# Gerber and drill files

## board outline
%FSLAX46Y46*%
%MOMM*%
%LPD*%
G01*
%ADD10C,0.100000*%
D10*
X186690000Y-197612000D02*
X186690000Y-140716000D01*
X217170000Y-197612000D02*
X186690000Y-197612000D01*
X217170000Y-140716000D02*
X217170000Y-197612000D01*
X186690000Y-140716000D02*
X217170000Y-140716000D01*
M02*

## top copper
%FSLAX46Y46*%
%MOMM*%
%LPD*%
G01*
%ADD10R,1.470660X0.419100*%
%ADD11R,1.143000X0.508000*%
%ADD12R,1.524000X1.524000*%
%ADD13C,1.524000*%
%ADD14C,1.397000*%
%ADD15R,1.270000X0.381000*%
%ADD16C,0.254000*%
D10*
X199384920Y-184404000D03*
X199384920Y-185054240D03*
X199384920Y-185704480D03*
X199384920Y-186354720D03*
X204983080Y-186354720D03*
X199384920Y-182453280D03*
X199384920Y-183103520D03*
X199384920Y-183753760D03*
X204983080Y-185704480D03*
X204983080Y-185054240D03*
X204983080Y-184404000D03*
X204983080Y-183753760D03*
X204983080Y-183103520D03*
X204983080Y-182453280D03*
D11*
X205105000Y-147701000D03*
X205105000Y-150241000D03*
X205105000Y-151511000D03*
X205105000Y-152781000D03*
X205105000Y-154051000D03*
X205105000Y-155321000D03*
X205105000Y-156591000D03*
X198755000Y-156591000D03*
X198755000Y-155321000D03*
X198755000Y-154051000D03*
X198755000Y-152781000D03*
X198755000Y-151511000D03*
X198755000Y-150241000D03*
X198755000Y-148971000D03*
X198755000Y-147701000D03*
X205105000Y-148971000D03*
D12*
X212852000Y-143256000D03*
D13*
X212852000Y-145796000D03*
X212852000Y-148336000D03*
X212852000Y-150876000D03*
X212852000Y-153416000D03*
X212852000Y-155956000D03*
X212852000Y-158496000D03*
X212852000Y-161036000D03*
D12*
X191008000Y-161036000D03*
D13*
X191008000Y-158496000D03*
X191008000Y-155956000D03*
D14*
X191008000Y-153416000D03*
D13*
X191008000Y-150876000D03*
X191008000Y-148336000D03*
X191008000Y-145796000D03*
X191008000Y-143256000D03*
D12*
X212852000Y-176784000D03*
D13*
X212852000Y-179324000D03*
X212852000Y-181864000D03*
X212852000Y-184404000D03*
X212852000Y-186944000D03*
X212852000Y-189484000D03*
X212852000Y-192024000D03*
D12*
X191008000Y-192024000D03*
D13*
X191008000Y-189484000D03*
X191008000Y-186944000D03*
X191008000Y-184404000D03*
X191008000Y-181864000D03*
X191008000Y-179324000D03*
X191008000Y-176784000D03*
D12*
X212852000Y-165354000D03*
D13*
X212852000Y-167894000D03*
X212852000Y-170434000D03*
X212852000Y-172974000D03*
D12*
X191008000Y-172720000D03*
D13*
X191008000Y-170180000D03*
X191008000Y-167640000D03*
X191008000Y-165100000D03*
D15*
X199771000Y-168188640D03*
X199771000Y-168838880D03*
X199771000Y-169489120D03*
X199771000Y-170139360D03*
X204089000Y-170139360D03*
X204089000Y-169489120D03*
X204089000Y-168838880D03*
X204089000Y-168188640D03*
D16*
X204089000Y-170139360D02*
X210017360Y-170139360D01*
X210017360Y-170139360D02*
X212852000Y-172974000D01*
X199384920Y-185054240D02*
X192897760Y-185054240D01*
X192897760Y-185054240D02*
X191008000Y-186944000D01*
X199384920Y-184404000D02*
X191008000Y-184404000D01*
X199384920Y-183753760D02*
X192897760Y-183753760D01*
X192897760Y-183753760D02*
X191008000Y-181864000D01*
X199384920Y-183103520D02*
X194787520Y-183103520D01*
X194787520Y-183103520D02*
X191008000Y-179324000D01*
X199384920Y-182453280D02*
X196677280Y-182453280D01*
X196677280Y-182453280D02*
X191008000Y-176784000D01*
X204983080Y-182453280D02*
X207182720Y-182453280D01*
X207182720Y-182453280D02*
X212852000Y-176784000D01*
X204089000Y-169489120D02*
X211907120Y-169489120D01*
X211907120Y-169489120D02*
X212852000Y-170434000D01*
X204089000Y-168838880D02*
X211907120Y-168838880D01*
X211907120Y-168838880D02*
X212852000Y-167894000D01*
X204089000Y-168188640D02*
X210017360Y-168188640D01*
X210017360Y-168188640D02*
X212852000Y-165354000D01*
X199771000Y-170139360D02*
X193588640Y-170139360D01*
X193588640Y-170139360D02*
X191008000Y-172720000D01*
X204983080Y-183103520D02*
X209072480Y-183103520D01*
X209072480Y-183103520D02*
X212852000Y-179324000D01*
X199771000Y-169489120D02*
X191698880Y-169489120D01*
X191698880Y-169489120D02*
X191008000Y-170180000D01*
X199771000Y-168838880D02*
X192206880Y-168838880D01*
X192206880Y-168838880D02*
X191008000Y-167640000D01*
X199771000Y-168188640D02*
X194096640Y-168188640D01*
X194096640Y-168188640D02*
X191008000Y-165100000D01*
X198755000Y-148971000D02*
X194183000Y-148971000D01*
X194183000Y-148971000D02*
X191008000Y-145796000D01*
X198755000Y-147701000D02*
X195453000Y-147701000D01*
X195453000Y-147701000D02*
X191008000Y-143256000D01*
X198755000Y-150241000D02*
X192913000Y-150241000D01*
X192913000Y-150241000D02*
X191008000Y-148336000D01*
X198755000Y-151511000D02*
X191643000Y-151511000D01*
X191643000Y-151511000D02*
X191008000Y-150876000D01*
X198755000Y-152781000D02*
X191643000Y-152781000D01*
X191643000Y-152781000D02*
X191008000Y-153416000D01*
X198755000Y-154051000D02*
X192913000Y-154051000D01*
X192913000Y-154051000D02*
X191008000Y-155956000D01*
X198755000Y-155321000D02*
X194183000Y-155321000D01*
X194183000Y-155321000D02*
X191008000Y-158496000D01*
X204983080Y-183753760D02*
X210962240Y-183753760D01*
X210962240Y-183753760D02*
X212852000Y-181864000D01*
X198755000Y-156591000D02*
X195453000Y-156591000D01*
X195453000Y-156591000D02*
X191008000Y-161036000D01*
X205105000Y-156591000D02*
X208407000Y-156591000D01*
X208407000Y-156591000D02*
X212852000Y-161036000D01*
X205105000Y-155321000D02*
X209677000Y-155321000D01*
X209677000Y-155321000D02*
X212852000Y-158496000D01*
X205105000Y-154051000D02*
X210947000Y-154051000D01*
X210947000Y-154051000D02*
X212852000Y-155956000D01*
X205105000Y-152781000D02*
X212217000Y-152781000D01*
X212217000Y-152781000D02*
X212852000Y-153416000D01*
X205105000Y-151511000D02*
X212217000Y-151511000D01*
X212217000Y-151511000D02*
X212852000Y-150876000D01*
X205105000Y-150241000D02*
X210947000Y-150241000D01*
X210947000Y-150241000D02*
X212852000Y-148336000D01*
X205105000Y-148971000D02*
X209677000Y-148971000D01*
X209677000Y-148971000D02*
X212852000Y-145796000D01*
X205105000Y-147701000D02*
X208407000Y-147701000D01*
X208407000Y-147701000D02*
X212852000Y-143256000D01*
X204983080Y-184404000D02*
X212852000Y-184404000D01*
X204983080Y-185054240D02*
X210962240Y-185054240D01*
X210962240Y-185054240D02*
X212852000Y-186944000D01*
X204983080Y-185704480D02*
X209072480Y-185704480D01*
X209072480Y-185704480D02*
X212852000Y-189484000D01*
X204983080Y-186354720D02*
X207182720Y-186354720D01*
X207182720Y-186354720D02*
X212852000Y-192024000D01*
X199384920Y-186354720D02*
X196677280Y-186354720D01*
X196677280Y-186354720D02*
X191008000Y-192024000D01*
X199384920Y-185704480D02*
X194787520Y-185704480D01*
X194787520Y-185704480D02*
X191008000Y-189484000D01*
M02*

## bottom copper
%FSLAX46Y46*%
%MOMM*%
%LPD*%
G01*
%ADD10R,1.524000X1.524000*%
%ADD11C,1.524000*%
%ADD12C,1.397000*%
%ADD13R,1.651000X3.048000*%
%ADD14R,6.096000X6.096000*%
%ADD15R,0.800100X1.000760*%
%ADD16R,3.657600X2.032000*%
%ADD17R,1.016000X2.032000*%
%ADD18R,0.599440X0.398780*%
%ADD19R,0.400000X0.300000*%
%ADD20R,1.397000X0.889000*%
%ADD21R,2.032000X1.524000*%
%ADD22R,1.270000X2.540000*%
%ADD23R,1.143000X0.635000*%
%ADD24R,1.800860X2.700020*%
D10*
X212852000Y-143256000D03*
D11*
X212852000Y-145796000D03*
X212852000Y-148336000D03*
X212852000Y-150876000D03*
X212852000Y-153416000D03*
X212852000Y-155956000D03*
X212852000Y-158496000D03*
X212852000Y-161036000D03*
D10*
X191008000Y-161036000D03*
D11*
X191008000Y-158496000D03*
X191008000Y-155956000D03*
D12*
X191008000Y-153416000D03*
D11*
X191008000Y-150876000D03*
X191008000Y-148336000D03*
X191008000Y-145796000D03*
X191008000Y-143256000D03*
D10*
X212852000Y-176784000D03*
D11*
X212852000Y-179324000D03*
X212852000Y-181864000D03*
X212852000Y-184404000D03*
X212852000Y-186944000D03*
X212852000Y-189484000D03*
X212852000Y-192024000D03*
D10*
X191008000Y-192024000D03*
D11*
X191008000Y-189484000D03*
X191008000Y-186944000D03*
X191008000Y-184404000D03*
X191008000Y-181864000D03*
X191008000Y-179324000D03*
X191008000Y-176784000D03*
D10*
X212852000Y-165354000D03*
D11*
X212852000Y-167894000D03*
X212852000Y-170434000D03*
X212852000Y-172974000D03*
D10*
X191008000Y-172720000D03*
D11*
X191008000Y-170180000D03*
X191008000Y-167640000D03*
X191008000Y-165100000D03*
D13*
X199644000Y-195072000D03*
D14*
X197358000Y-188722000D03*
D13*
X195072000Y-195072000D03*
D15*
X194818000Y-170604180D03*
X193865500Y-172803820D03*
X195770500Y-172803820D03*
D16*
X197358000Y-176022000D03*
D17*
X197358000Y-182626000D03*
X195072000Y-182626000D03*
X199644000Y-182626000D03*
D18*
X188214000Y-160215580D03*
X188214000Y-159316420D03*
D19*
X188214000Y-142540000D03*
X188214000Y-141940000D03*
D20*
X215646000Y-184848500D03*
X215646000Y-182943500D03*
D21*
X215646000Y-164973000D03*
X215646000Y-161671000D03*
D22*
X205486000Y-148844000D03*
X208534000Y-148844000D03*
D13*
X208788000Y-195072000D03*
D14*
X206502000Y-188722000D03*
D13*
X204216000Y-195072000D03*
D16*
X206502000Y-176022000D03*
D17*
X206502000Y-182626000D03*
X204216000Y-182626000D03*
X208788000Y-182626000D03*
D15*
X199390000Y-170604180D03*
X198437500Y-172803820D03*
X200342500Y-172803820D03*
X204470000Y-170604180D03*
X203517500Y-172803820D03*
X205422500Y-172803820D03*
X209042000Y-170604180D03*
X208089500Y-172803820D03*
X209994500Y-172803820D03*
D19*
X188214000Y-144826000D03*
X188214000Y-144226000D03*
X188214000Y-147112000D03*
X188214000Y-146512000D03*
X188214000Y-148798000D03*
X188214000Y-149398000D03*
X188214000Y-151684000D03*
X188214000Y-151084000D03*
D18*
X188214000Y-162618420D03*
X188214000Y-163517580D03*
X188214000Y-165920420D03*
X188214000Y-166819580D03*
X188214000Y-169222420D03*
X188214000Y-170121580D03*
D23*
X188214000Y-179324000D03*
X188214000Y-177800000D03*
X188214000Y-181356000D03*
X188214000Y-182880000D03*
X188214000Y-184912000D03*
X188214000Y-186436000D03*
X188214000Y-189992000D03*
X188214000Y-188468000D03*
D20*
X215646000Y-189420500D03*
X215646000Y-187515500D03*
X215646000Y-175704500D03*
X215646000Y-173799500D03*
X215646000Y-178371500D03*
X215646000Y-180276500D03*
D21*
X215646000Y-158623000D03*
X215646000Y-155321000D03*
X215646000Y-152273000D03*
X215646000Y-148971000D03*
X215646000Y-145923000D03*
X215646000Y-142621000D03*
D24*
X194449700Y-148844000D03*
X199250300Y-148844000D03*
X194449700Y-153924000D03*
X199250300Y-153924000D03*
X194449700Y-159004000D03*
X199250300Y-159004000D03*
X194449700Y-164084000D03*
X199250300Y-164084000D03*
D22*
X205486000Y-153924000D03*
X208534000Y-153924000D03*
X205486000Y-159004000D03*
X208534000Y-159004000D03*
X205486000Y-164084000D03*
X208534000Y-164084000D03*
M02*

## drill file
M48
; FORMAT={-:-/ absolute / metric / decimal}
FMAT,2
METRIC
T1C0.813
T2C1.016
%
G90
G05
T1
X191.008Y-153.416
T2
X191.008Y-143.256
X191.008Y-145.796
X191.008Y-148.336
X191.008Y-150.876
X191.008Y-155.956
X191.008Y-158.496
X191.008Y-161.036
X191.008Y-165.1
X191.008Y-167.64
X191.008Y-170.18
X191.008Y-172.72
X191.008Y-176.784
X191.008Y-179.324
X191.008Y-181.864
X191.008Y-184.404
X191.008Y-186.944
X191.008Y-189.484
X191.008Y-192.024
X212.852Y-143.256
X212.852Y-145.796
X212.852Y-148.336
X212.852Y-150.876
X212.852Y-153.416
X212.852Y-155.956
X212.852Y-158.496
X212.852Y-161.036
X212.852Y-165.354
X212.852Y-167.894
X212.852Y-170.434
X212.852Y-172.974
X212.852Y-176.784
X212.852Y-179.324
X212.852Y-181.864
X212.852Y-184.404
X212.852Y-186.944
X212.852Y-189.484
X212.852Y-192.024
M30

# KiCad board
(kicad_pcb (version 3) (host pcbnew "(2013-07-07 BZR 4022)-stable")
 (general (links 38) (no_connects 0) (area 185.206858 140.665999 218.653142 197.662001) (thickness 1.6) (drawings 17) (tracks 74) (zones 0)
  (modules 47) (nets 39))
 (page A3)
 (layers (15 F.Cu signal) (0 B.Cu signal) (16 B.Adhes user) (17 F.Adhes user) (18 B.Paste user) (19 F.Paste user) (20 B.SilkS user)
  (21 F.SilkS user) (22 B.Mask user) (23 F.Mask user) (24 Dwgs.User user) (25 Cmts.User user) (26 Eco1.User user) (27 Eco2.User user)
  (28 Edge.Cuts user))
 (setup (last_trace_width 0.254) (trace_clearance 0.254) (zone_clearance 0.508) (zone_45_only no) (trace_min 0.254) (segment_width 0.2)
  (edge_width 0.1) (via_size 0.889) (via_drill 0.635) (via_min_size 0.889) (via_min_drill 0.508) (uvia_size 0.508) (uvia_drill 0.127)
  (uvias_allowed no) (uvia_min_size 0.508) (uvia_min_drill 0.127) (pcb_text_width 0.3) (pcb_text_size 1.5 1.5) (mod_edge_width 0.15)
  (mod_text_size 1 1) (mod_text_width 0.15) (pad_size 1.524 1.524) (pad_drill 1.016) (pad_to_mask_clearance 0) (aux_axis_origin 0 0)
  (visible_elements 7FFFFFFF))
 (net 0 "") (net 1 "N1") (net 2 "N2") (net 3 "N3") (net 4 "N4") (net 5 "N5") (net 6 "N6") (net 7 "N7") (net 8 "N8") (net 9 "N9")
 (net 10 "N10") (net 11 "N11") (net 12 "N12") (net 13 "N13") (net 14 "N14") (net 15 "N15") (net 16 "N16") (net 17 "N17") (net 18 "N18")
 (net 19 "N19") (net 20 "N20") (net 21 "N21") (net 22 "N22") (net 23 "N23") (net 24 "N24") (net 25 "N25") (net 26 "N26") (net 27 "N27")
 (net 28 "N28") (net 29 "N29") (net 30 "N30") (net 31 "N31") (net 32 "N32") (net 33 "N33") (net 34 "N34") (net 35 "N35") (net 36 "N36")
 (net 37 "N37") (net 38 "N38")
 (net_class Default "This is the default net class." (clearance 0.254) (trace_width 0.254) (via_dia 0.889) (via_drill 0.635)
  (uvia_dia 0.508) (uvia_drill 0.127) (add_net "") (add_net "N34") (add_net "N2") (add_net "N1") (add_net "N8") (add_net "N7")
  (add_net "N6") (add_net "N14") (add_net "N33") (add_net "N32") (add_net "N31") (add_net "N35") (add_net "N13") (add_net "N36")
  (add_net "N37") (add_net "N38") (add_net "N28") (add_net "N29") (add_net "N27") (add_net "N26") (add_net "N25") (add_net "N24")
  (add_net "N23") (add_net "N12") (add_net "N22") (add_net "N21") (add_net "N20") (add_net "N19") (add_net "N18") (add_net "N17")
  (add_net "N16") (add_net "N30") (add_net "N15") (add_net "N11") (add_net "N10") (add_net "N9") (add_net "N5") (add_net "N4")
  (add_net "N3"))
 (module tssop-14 (layer F.Cu) (at 202.184 184.404 270)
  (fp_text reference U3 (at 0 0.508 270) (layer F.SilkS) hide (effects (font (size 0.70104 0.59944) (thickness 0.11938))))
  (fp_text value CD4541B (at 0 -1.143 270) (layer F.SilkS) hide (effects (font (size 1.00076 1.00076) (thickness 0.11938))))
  (pad 4 smd rect (at 0 2.79908 270) (size 0.4191 1.47066) (layers F.Cu F.Paste F.Mask) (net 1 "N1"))
  (pad 5 smd rect (at 0.65024 2.79908 270) (size 0.4191 1.47066) (layers F.Cu F.Paste F.Mask) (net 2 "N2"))
  (pad 6 smd rect (at 1.30048 2.79908 270) (size 0.4191 1.47066) (layers F.Cu F.Paste F.Mask) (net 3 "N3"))
  (pad 7 smd rect (at 1.95072 2.79908 270) (size 0.4191 1.47066) (layers F.Cu F.Paste F.Mask) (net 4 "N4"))
  (pad 8 smd rect (at 1.95072 -2.79908 270) (size 0.4191 1.47066) (layers F.Cu F.Paste F.Mask) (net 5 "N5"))
  (pad 1 smd rect (at -1.95072 2.79908 270) (size 0.4191 1.47066) (layers F.Cu F.Paste F.Mask) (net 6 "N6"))
  (pad 2 smd rect (at -1.30048 2.79908 270) (size 0.4191 1.47066) (layers F.Cu F.Paste F.Mask) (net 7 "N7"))
  (pad 3 smd rect (at -0.65024 2.79908 270) (size 0.4191 1.47066) (layers F.Cu F.Paste F.Mask) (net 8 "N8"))
  (pad 9 smd rect (at 1.30048 -2.79908 270) (size 0.4191 1.47066) (layers F.Cu F.Paste F.Mask) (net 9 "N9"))
  (pad 10 smd rect (at 0.65024 -2.79908 270) (size 0.4191 1.47066) (layers F.Cu F.Paste F.Mask) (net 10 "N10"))
  (pad 11 smd rect (at 0 -2.79908 270) (size 0.4191 1.47066) (layers F.Cu F.Paste F.Mask) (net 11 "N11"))
  (pad 12 smd rect (at -0.65024 -2.79908 270) (size 0.4191 1.47066) (layers F.Cu F.Paste F.Mask) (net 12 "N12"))
  (pad 13 smd rect (at -1.30048 -2.79908 270) (size 0.4191 1.47066) (layers F.Cu F.Paste F.Mask) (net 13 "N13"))
  (pad 14 smd rect (at -1.95072 -2.79908 270) (size 0.4191 1.47066) (layers F.Cu F.Paste F.Mask) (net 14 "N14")))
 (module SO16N (layer F.Cu) (at 201.93 152.146 270)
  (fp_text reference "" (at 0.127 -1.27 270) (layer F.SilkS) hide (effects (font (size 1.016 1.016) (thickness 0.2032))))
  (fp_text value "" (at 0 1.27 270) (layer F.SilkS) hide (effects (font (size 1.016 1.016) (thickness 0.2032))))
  (pad 16 smd rect (at -4.445 -3.175 270) (size 0.508 1.143) (layers F.Cu F.Paste F.Mask) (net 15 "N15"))
  (pad 14 smd rect (at -1.905 -3.175 270) (size 0.508 1.143) (layers F.Cu F.Paste F.Mask) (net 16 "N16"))
  (pad 13 smd rect (at -0.635 -3.175 270) (size 0.508 1.143) (layers F.Cu F.Paste F.Mask) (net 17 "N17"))
  (pad 12 smd rect (at 0.635 -3.175 270) (size 0.508 1.143) (layers F.Cu F.Paste F.Mask) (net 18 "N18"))
  (pad 11 smd rect (at 1.905 -3.175 270) (size 0.508 1.143) (layers F.Cu F.Paste F.Mask) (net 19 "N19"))
  (pad 10 smd rect (at 3.175 -3.175 270) (size 0.508 1.143) (layers F.Cu F.Paste F.Mask) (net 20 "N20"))
  (pad 9 smd rect (at 4.445 -3.175 270) (size 0.508 1.143) (layers F.Cu F.Paste F.Mask) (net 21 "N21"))
  (pad 8 smd rect (at 4.445 3.175 270) (size 0.508 1.143) (layers F.Cu F.Paste F.Mask) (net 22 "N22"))
  (pad 7 smd rect (at 3.175 3.175 270) (size 0.508 1.143) (layers F.Cu F.Paste F.Mask) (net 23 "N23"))
  (pad 6 smd rect (at 1.905 3.175 270) (size 0.508 1.143) (layers F.Cu F.Paste F.Mask) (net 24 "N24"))
  (pad 5 smd rect (at 0.635 3.175 270) (size 0.508 1.143) (layers F.Cu F.Paste F.Mask) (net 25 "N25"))
  (pad 4 smd rect (at -0.635 3.175 270) (size 0.508 1.143) (layers F.Cu F.Paste F.Mask) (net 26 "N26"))
  (pad 3 smd rect (at -1.905 3.175 270) (size 0.508 1.143) (layers F.Cu F.Paste F.Mask) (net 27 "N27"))
  (pad 2 smd rect (at -3.175 3.175 270) (size 0.508 1.143) (layers F.Cu F.Paste F.Mask) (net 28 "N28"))
  (pad 1 smd rect (at -4.445 3.175 270) (size 0.508 1.143) (layers F.Cu F.Paste F.Mask) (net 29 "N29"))
  (pad 15 smd rect (at -3.175 -3.175 270) (size 0.508 1.143) (layers F.Cu F.Paste F.Mask) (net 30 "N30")))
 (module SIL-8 (layer F.Cu) (at 212.852 152.146 270)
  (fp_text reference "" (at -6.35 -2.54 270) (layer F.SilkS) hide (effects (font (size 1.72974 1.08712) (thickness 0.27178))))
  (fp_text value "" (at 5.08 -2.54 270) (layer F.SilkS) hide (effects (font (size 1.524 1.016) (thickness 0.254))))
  (pad 1 thru_hole rect (at -8.89 0 270) (size 1.524 1.524) (drill 1.016) (layers *.Cu *.Mask F.SilkS) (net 15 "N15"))
  (pad 2 thru_hole circle (at -6.35 0 270) (size 1.524 1.524) (drill 1.016) (layers *.Cu *.Mask F.SilkS) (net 30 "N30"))
  (pad 3 thru_hole circle (at -3.81 0 270) (size 1.524 1.524) (drill 1.016) (layers *.Cu *.Mask F.SilkS) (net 16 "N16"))
  (pad 4 thru_hole circle (at -1.27 0 270) (size 1.524 1.524) (drill 1.016) (layers *.Cu *.Mask F.SilkS) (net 17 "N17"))
  (pad 5 thru_hole circle (at 1.27 0 270) (size 1.524 1.524) (drill 1.016) (layers *.Cu *.Mask F.SilkS) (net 18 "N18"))
  (pad 6 thru_hole circle (at 3.81 0 270) (size 1.524 1.524) (drill 1.016) (layers *.Cu *.Mask F.SilkS) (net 19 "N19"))
  (pad 7 thru_hole circle (at 6.35 0 270) (size 1.524 1.524) (drill 1.016) (layers *.Cu *.Mask F.SilkS) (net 20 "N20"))
  (pad 8 thru_hole circle (at 8.89 0 270) (size 1.524 1.524) (drill 1.016) (layers *.Cu *.Mask F.SilkS) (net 21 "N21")))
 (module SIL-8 (layer F.Cu) (at 191.008 152.146 90)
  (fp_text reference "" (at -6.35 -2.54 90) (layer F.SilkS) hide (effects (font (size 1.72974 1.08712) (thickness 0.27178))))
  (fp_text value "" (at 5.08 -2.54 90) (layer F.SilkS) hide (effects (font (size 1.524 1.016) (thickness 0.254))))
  (pad 1 thru_hole rect (at -8.89 0 90) (size 1.524 1.524) (drill 1.016) (layers *.Cu *.Mask F.SilkS) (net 22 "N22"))
  (pad 2 thru_hole circle (at -6.35 0 90) (size 1.524 1.524) (drill 1.016) (layers *.Cu *.Mask F.SilkS) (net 23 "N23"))
  (pad 3 thru_hole circle (at -3.81 0 90) (size 1.524 1.524) (drill 1.016) (layers *.Cu *.Mask F.SilkS) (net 24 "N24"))
  (pad 4 thru_hole circle (at -1.27 0 90) (size 1.397 1.397) (drill 0.8128) (layers *.Cu *.Mask F.SilkS) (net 25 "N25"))
  (pad 5 thru_hole circle (at 1.27 0 90) (size 1.524 1.524) (drill 1.016) (layers *.Cu *.Mask F.SilkS) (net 26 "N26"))
  (pad 6 thru_hole circle (at 3.81 0 90) (size 1.524 1.524) (drill 1.016) (layers *.Cu *.Mask F.SilkS) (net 27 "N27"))
  (pad 7 thru_hole circle (at 6.35 0 90) (size 1.524 1.524) (drill 1.016) (layers *.Cu *.Mask F.SilkS) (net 28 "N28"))
  (pad 8 thru_hole circle (at 8.89 0 90) (size 1.524 1.524) (drill 1.016) (layers *.Cu *.Mask F.SilkS) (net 29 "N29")))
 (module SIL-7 (layer F.Cu) (at 212.852 184.404 270)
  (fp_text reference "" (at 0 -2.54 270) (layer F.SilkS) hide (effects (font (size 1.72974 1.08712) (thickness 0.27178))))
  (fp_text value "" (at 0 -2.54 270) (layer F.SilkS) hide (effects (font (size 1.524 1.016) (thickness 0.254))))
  (pad 1 thru_hole rect (at -7.62 0 270) (size 1.524 1.524) (drill 1.016) (layers *.Cu *.Mask F.SilkS) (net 14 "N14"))
  (pad 2 thru_hole circle (at -5.08 0 270) (size 1.524 1.524) (drill 1.016) (layers *.Cu *.SilkS *.Mask) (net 13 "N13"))
  (pad 3 thru_hole circle (at -2.54 0 270) (size 1.524 1.524) (drill 1.016) (layers *.Cu *.SilkS *.Mask) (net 12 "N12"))
  (pad 4 thru_hole circle (at 0 0 270) (size 1.524 1.524) (drill 1.016) (layers *.Cu *.SilkS *.Mask) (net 11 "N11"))
  (pad 5 thru_hole circle (at 2.54 0 270) (size 1.524 1.524) (drill 1.016) (layers *.Cu *.SilkS *.Mask) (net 10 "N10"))
  (pad 6 thru_hole circle (at 5.08 0 270) (size 1.524 1.524) (drill 1.016) (layers *.Cu *.SilkS *.Mask) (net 9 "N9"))
  (pad 7 thru_hole circle (at 7.62 0 270) (size 1.524 1.524) (drill 1.016) (layers *.Cu *.SilkS *.Mask) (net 5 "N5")))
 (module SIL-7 (layer F.Cu) (at 191.008 184.404 90)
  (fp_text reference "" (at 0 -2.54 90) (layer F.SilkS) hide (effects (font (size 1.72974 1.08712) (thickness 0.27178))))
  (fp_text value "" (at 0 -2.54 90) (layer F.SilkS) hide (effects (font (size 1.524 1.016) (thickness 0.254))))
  (pad 1 thru_hole rect (at -7.62 0 90) (size 1.524 1.524) (drill 1.016) (layers *.Cu *.Mask F.SilkS) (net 4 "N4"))
  (pad 2 thru_hole circle (at -5.08 0 90) (size 1.524 1.524) (drill 1.016) (layers *.Cu *.SilkS *.Mask) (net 3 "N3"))
  (pad 3 thru_hole circle (at -2.54 0 90) (size 1.524 1.524) (drill 1.016) (layers *.Cu *.SilkS *.Mask) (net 2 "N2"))
  (pad 4 thru_hole circle (at 0 0 90) (size 1.524 1.524) (drill 1.016) (layers *.Cu *.SilkS *.Mask) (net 1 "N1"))
  (pad 5 thru_hole circle (at 2.54 0 90) (size 1.524 1.524) (drill 1.016) (layers *.Cu *.SilkS *.Mask) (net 8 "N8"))
  (pad 6 thru_hole circle (at 5.08 0 90) (size 1.524 1.524) (drill 1.016) (layers *.Cu *.SilkS *.Mask) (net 7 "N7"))
  (pad 7 thru_hole circle (at 7.62 0 90) (size 1.524 1.524) (drill 1.016) (layers *.Cu *.SilkS *.Mask) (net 6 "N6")))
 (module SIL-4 (layer F.Cu) (at 212.852 169.164 270)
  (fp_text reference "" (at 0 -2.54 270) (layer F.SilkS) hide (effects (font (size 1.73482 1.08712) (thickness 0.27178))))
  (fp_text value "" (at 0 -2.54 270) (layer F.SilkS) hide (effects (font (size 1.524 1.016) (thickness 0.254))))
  (pad 1 thru_hole rect (at -3.81 0 270) (size 1.524 1.524) (drill 1.016) (layers *.Cu *.Mask F.SilkS) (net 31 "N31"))
  (pad 2 thru_hole circle (at -1.27 0 270) (size 1.524 1.524) (drill 1.016) (layers *.Cu *.Mask F.SilkS) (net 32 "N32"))
  (pad 3 thru_hole circle (at 1.27 0 270) (size 1.524 1.524) (drill 1.016) (layers *.Cu *.Mask F.SilkS) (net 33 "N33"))
  (pad 4 thru_hole circle (at 3.81 0 270) (size 1.524 1.524) (drill 1.016) (layers *.Cu *.Mask F.SilkS) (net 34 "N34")))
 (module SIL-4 (layer F.Cu) (at 191.008 168.91 90)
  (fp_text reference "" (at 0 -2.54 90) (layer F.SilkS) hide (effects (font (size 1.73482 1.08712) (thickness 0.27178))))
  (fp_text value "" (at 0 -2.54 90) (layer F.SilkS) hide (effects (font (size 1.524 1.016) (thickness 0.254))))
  (pad 1 thru_hole rect (at -3.81 0 90) (size 1.524 1.524) (drill 1.016) (layers *.Cu *.Mask F.SilkS) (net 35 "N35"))
  (pad 2 thru_hole circle (at -1.27 0 90) (size 1.524 1.524) (drill 1.016) (layers *.Cu *.Mask F.SilkS) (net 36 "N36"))
  (pad 3 thru_hole circle (at 1.27 0 90) (size 1.524 1.524) (drill 1.016) (layers *.Cu *.Mask F.SilkS) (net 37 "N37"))
  (pad 4 thru_hole circle (at 3.81 0 90) (size 1.524 1.524) (drill 1.016) (layers *.Cu *.Mask F.SilkS) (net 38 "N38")))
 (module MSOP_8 (layer F.Cu) (at 201.93 169.164 270)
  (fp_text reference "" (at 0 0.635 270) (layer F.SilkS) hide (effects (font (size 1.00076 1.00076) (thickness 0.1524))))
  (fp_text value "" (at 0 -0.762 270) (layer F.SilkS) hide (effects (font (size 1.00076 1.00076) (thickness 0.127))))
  (pad 1 smd rect (at -0.97536 2.159 270) (size 0.381 1.27) (layers F.Cu F.Paste F.Mask) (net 38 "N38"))
  (pad 2 smd rect (at -0.32512 2.159 270) (size 0.381 1.27) (layers F.Cu F.Paste F.Mask) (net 37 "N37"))
  (pad 3 smd rect (at 0.32512 2.159 270) (size 0.381 1.27) (layers F.Cu F.Paste F.Mask) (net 36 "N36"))
  (pad 4 smd rect (at 0.97536 2.159 270) (size 0.381 1.27) (layers F.Cu F.Paste F.Mask) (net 35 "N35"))
  (pad 5 smd rect (at 0.97536 -2.159 270) (size 0.381 1.27) (layers F.Cu F.Paste F.Mask) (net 34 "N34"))
  (pad 6 smd rect (at 0.32512 -2.159 270) (size 0.381 1.27) (layers F.Cu F.Paste F.Mask) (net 33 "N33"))
  (pad 7 smd rect (at -0.32512 -2.159 270) (size 0.381 1.27) (layers F.Cu F.Paste F.Mask) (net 32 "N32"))
  (pad 8 smd rect (at -0.97536 -2.159 270) (size 0.381 1.27) (layers F.Cu F.Paste F.Mask) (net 31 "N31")))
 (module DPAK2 (layer B.Cu) (at 197.358 195.072 180)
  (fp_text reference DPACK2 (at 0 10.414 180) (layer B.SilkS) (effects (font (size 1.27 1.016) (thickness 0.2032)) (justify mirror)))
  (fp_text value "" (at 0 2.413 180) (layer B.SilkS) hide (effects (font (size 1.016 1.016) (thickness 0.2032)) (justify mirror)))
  (pad 1 smd rect (at -2.286 0 180) (size 1.651 3.048) (layers B.Cu B.Paste B.Mask))
  (pad 2 smd rect (at 0 6.35 180) (size 6.096 6.096) (layers B.Cu B.Paste B.Mask))
  (pad 3 smd rect (at 2.286 0 180) (size 1.651 3.048) (layers B.Cu B.Paste B.Mask)))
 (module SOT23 (layer B.Cu) (at 194.818 171.704 180)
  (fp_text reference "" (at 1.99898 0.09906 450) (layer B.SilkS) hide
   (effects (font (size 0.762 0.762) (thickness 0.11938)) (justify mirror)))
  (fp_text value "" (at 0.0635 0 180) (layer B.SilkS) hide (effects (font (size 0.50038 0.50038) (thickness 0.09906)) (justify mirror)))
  (pad 3 smd rect (at 0 1.09982 180) (size 0.8001 1.00076) (layers B.Cu B.Paste B.Mask))
  (pad 2 smd rect (at 0.9525 -1.09982 180) (size 0.8001 1.00076) (layers B.Cu B.Paste B.Mask))
  (pad 1 smd rect (at -0.9525 -1.09982 180) (size 0.8001 1.00076) (layers B.Cu B.Paste B.Mask)))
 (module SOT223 (layer B.Cu) (at 197.358 179.324 180)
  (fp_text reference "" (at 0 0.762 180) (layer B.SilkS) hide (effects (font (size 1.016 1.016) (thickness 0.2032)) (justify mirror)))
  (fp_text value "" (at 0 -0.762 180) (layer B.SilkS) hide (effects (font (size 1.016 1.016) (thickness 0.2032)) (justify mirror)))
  (pad 4 smd rect (at 0 3.302 180) (size 3.6576 2.032) (layers B.Cu B.Paste B.Mask))
  (pad 2 smd rect (at 0 -3.302 180) (size 1.016 2.032) (layers B.Cu B.Paste B.Mask))
  (pad 3 smd rect (at 2.286 -3.302 180) (size 1.016 2.032) (layers B.Cu B.Paste B.Mask))
  (pad 1 smd rect (at -2.286 -3.302 180) (size 1.016 2.032) (layers B.Cu B.Paste B.Mask)))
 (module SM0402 (layer B.Cu) (at 188.214 159.766 90)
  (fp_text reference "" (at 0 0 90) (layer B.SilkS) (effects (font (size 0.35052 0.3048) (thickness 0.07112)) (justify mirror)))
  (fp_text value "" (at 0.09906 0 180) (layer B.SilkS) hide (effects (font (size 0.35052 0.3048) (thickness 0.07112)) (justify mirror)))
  (pad 1 smd rect (at -0.44958 0 90) (size 0.39878 0.59944) (layers B.Cu B.Paste B.Mask))
  (pad 2 smd rect (at 0.44958 0 90) (size 0.39878 0.59944) (layers B.Cu B.Paste B.Mask)))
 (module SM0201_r (layer B.Cu) (at 188.214 142.24 90)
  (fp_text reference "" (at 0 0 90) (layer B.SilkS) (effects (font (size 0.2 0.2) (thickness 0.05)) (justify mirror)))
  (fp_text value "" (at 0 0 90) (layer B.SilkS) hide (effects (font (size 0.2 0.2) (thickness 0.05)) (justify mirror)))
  (pad 1 smd rect (at -0.3 0 90) (size 0.3 0.4) (layers B.Cu B.Paste B.Mask))
  (pad 2 smd rect (at 0.3 0 90) (size 0.3 0.4) (layers B.Cu B.Paste B.Mask)))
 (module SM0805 (layer B.Cu) (at 215.646 183.896 90)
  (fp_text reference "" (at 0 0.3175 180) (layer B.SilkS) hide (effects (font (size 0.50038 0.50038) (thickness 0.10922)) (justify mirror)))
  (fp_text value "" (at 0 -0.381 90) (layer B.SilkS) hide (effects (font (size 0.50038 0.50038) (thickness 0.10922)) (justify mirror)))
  (pad 1 smd rect (at -0.9525 0 90) (size 0.889 1.397) (layers B.Cu B.Paste B.Mask))
  (pad 2 smd rect (at 0.9525 0 90) (size 0.889 1.397) (layers B.Cu B.Paste B.Mask)))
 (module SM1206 (layer B.Cu) (at 215.646 163.322 90)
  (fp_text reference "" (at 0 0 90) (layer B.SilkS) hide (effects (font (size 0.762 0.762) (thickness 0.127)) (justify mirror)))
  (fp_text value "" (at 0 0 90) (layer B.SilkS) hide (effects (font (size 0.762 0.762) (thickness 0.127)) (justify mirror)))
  (pad 1 smd rect (at -1.651 0 90) (size 1.524 2.032) (layers B.Cu B.Paste B.Mask))
  (pad 2 smd rect (at 1.651 0 90) (size 1.524 2.032) (layers B.Cu B.Paste B.Mask)))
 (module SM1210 (layer B.Cu) (at 207.01 148.844)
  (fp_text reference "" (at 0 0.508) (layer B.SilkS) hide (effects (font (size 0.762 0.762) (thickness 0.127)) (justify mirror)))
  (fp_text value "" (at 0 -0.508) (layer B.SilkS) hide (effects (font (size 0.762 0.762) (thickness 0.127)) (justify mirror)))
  (pad 1 smd rect (at -1.524 0) (size 1.27 2.54) (layers B.Cu B.Paste B.Mask))
  (pad 2 smd rect (at 1.524 0) (size 1.27 2.54) (layers B.Cu B.Paste B.Mask)))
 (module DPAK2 (layer B.Cu) (at 206.502 195.072 180)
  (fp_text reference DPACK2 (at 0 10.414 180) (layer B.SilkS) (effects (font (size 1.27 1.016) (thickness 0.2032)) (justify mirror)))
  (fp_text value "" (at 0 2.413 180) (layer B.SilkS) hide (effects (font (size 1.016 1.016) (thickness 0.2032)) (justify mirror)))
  (pad 1 smd rect (at -2.286 0 180) (size 1.651 3.048) (layers B.Cu B.Paste B.Mask))
  (pad 2 smd rect (at 0 6.35 180) (size 6.096 6.096) (layers B.Cu B.Paste B.Mask))
  (pad 3 smd rect (at 2.286 0 180) (size 1.651 3.048) (layers B.Cu B.Paste B.Mask)))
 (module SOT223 (layer B.Cu) (at 206.502 179.324 180)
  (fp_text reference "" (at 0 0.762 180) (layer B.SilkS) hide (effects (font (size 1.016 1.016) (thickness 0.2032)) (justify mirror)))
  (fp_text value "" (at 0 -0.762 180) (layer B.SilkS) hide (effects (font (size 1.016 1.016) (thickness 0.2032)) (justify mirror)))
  (pad 4 smd rect (at 0 3.302 180) (size 3.6576 2.032) (layers B.Cu B.Paste B.Mask))
  (pad 2 smd rect (at 0 -3.302 180) (size 1.016 2.032) (layers B.Cu B.Paste B.Mask))
  (pad 3 smd rect (at 2.286 -3.302 180) (size 1.016 2.032) (layers B.Cu B.Paste B.Mask))
  (pad 1 smd rect (at -2.286 -3.302 180) (size 1.016 2.032) (layers B.Cu B.Paste B.Mask)))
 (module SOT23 (layer B.Cu) (at 199.39 171.704 180)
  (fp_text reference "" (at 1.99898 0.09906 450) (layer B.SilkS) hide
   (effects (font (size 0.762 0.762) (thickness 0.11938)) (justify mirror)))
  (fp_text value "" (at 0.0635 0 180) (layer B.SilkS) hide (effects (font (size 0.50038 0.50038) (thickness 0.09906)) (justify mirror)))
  (pad 3 smd rect (at 0 1.09982 180) (size 0.8001 1.00076) (layers B.Cu B.Paste B.Mask))
  (pad 2 smd rect (at 0.9525 -1.09982 180) (size 0.8001 1.00076) (layers B.Cu B.Paste B.Mask))
  (pad 1 smd rect (at -0.9525 -1.09982 180) (size 0.8001 1.00076) (layers B.Cu B.Paste B.Mask)))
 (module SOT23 (layer B.Cu) (at 204.47 171.704 180)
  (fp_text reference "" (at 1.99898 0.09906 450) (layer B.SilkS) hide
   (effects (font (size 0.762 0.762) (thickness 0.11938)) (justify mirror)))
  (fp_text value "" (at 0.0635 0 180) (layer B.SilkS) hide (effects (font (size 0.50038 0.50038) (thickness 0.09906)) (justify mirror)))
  (pad 3 smd rect (at 0 1.09982 180) (size 0.8001 1.00076) (layers B.Cu B.Paste B.Mask))
  (pad 2 smd rect (at 0.9525 -1.09982 180) (size 0.8001 1.00076) (layers B.Cu B.Paste B.Mask))
  (pad 1 smd rect (at -0.9525 -1.09982 180) (size 0.8001 1.00076) (layers B.Cu B.Paste B.Mask)))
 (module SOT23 (layer B.Cu) (at 209.042 171.704 180)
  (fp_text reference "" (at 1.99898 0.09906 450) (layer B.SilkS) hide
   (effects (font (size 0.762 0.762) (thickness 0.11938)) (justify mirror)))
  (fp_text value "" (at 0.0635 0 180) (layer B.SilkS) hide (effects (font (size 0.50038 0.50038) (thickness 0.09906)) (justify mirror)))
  (pad 3 smd rect (at 0 1.09982 180) (size 0.8001 1.00076) (layers B.Cu B.Paste B.Mask))
  (pad 2 smd rect (at 0.9525 -1.09982 180) (size 0.8001 1.00076) (layers B.Cu B.Paste B.Mask))
  (pad 1 smd rect (at -0.9525 -1.09982 180) (size 0.8001 1.00076) (layers B.Cu B.Paste B.Mask)))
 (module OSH (layer F.Cu) (at 201.93 189.992)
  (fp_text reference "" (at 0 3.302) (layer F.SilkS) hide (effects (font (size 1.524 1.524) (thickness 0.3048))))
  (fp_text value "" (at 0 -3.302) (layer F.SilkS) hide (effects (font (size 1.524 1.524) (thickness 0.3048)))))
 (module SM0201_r (layer B.Cu) (at 188.214 144.526 90)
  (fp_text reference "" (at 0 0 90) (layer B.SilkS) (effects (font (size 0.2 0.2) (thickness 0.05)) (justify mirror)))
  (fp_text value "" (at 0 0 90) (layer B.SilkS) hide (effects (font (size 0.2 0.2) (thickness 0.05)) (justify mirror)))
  (pad 1 smd rect (at -0.3 0 90) (size 0.3 0.4) (layers B.Cu B.Paste B.Mask))
  (pad 2 smd rect (at 0.3 0 90) (size 0.3 0.4) (layers B.Cu B.Paste B.Mask)))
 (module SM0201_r (layer B.Cu) (at 188.214 146.812 90)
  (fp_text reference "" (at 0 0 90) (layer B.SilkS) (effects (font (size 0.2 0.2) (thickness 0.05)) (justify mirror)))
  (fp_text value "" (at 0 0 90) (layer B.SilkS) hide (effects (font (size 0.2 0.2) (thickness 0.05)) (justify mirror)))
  (pad 1 smd rect (at -0.3 0 90) (size 0.3 0.4) (layers B.Cu B.Paste B.Mask))
  (pad 2 smd rect (at 0.3 0 90) (size 0.3 0.4) (layers B.Cu B.Paste B.Mask)))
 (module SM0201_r (layer B.Cu) (at 188.214 149.098 270)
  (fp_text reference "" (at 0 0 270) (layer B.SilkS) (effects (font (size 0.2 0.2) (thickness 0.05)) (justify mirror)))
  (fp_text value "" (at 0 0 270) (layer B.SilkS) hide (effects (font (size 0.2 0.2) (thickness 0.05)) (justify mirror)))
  (pad 1 smd rect (at -0.3 0 270) (size 0.3 0.4) (layers B.Cu B.Paste B.Mask))
  (pad 2 smd rect (at 0.3 0 270) (size 0.3 0.4) (layers B.Cu B.Paste B.Mask)))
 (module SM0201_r (layer B.Cu) (at 188.214 151.384 90)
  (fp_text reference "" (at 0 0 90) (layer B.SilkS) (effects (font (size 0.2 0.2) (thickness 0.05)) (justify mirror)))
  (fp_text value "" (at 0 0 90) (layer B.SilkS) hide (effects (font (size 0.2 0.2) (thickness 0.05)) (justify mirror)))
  (pad 1 smd rect (at -0.3 0 90) (size 0.3 0.4) (layers B.Cu B.Paste B.Mask))
  (pad 2 smd rect (at 0.3 0 90) (size 0.3 0.4) (layers B.Cu B.Paste B.Mask)))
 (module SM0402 (layer B.Cu) (at 188.214 163.068 270)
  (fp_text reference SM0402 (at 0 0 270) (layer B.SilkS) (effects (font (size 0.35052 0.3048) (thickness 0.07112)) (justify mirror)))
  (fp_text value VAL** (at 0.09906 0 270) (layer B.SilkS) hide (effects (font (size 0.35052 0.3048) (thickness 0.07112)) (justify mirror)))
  (pad 1 smd rect (at -0.44958 0 270) (size 0.39878 0.59944) (layers B.Cu B.Paste B.Mask))
  (pad 2 smd rect (at 0.44958 0 270) (size 0.39878 0.59944) (layers B.Cu B.Paste B.Mask)))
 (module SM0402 (layer B.Cu) (at 188.214 166.37 270)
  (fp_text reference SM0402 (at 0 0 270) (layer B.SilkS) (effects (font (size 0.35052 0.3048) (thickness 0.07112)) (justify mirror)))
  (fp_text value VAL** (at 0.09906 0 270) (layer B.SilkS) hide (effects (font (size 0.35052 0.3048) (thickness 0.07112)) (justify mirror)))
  (pad 1 smd rect (at -0.44958 0 270) (size 0.39878 0.59944) (layers B.Cu B.Paste B.Mask))
  (pad 2 smd rect (at 0.44958 0 270) (size 0.39878 0.59944) (layers B.Cu B.Paste B.Mask)))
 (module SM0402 (layer B.Cu) (at 188.214 169.672 270)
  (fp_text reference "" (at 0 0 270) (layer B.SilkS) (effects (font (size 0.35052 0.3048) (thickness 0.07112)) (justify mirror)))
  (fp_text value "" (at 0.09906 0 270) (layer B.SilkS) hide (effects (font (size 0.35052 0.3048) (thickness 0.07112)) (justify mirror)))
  (pad 1 smd rect (at -0.44958 0 270) (size 0.39878 0.59944) (layers B.Cu B.Paste B.Mask))
  (pad 2 smd rect (at 0.44958 0 270) (size 0.39878 0.59944) (layers B.Cu B.Paste B.Mask)))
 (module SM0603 (layer B.Cu) (at 188.214 178.562 90)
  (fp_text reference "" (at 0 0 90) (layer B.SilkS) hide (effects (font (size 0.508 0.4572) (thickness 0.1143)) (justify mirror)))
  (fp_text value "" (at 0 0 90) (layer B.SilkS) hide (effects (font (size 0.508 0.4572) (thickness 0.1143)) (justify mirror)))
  (pad 1 smd rect (at -0.762 0 90) (size 0.635 1.143) (layers B.Cu B.Paste B.Mask))
  (pad 2 smd rect (at 0.762 0 90) (size 0.635 1.143) (layers B.Cu B.Paste B.Mask)))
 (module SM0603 (layer B.Cu) (at 188.214 182.118 270)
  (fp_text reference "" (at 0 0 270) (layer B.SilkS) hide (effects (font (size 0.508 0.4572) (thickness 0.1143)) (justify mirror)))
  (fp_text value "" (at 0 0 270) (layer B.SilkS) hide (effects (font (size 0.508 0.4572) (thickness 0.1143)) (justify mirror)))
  (pad 1 smd rect (at -0.762 0 270) (size 0.635 1.143) (layers B.Cu B.Paste B.Mask))
  (pad 2 smd rect (at 0.762 0 270) (size 0.635 1.143) (layers B.Cu B.Paste B.Mask)))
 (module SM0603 (layer B.Cu) (at 188.214 185.674 270)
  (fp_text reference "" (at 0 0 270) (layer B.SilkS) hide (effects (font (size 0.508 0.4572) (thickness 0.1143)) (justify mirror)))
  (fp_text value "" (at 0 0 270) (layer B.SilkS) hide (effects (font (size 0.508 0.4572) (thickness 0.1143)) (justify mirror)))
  (pad 1 smd rect (at -0.762 0 270) (size 0.635 1.143) (layers B.Cu B.Paste B.Mask))
  (pad 2 smd rect (at 0.762 0 270) (size 0.635 1.143) (layers B.Cu B.Paste B.Mask)))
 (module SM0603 (layer B.Cu) (at 188.214 189.23 90)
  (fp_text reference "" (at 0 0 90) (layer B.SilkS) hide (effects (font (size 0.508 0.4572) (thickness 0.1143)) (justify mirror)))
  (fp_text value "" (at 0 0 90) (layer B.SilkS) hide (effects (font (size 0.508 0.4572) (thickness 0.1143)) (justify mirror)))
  (pad 1 smd rect (at -0.762 0 90) (size 0.635 1.143) (layers B.Cu B.Paste B.Mask))
  (pad 2 smd rect (at 0.762 0 90) (size 0.635 1.143) (layers B.Cu B.Paste B.Mask)))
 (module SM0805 (layer B.Cu) (at 215.646 188.468 90)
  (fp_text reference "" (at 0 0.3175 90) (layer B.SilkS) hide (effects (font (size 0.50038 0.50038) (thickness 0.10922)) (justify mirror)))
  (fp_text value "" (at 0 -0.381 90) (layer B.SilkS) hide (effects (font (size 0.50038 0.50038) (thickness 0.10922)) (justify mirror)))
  (pad 1 smd rect (at -0.9525 0 90) (size 0.889 1.397) (layers B.Cu B.Paste B.Mask))
  (pad 2 smd rect (at 0.9525 0 90) (size 0.889 1.397) (layers B.Cu B.Paste B.Mask)))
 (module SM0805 (layer B.Cu) (at 215.646 174.752 90)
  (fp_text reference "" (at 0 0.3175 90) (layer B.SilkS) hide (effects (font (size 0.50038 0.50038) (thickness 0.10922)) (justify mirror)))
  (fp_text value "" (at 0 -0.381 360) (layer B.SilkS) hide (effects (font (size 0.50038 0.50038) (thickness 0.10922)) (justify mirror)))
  (pad 1 smd rect (at -0.9525 0 90) (size 0.889 1.397) (layers B.Cu B.Paste B.Mask))
  (pad 2 smd rect (at 0.9525 0 90) (size 0.889 1.397) (layers B.Cu B.Paste B.Mask)))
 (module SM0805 (layer B.Cu) (at 215.646 179.324 270)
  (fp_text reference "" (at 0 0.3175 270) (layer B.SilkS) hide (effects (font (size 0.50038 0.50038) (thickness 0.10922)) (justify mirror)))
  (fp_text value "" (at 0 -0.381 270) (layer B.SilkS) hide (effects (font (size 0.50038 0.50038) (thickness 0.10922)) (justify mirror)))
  (pad 1 smd rect (at -0.9525 0 270) (size 0.889 1.397) (layers B.Cu B.Paste B.Mask))
  (pad 2 smd rect (at 0.9525 0 270) (size 0.889 1.397) (layers B.Cu B.Paste B.Mask)))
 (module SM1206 (layer B.Cu) (at 215.646 156.972 90)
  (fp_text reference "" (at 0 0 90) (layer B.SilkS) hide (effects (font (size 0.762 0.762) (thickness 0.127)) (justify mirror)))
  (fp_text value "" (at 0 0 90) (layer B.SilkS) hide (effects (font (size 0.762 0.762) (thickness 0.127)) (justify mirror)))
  (pad 1 smd rect (at -1.651 0 90) (size 1.524 2.032) (layers B.Cu B.Paste B.Mask))
  (pad 2 smd rect (at 1.651 0 90) (size 1.524 2.032) (layers B.Cu B.Paste B.Mask)))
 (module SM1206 (layer B.Cu) (at 215.646 150.622 90)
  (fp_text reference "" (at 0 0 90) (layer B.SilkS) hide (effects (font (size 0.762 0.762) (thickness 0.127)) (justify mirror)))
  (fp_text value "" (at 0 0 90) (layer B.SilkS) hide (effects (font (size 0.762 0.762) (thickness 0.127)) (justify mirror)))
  (pad 1 smd rect (at -1.651 0 90) (size 1.524 2.032) (layers B.Cu B.Paste B.Mask))
  (pad 2 smd rect (at 1.651 0 90) (size 1.524 2.032) (layers B.Cu B.Paste B.Mask)))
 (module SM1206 (layer B.Cu) (at 215.646 144.272 90)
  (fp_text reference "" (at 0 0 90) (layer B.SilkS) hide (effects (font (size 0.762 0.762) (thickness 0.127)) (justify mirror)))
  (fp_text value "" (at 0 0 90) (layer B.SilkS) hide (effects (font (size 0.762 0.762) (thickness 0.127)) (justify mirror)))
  (pad 1 smd rect (at -1.651 0 90) (size 1.524 2.032) (layers B.Cu B.Paste B.Mask))
  (pad 2 smd rect (at 1.651 0 90) (size 1.524 2.032) (layers B.Cu B.Paste B.Mask)))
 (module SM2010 (layer B.Cu) (at 196.85 148.844)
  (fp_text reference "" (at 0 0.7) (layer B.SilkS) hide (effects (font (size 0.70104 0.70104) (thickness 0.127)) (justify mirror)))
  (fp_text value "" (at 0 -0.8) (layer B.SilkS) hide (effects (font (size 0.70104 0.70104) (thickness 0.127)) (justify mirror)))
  (pad 1 smd rect (at -2.4003 0) (size 1.80086 2.70002) (layers B.Cu B.Paste B.Mask))
  (pad 2 smd rect (at 2.4003 0) (size 1.80086 2.70002) (layers B.Cu B.Paste B.Mask)))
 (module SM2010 (layer B.Cu) (at 196.85 153.924)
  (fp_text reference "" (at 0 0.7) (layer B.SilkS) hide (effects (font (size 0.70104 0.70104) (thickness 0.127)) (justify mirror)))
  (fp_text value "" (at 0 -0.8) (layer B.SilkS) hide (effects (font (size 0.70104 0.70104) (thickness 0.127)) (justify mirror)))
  (pad 1 smd rect (at -2.4003 0) (size 1.80086 2.70002) (layers B.Cu B.Paste B.Mask))
  (pad 2 smd rect (at 2.4003 0) (size 1.80086 2.70002) (layers B.Cu B.Paste B.Mask)))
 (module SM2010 (layer B.Cu) (at 196.85 159.004)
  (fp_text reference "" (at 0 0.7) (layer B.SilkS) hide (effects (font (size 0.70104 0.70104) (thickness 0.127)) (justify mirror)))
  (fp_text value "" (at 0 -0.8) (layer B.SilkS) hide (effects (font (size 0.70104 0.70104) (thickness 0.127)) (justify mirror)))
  (pad 1 smd rect (at -2.4003 0) (size 1.80086 2.70002) (layers B.Cu B.Paste B.Mask))
  (pad 2 smd rect (at 2.4003 0) (size 1.80086 2.70002) (layers B.Cu B.Paste B.Mask)))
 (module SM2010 (layer B.Cu) (at 196.85 164.084)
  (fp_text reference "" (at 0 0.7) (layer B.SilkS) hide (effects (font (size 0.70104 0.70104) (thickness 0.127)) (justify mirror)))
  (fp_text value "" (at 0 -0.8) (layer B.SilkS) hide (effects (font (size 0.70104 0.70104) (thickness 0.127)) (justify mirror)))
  (pad 1 smd rect (at -2.4003 0) (size 1.80086 2.70002) (layers B.Cu B.Paste B.Mask))
  (pad 2 smd rect (at 2.4003 0) (size 1.80086 2.70002) (layers B.Cu B.Paste B.Mask)))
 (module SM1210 (layer B.Cu) (at 207.01 153.924)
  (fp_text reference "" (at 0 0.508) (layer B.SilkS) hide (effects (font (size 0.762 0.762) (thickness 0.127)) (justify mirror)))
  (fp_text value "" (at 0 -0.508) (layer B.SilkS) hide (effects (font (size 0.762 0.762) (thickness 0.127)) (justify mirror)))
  (pad 1 smd rect (at -1.524 0) (size 1.27 2.54) (layers B.Cu B.Paste B.Mask))
  (pad 2 smd rect (at 1.524 0) (size 1.27 2.54) (layers B.Cu B.Paste B.Mask)))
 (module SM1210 (layer B.Cu) (at 207.01 159.004)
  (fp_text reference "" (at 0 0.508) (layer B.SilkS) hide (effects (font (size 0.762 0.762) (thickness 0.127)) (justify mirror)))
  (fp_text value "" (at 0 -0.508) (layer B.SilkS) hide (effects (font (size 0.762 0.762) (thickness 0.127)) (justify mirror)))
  (pad 1 smd rect (at -1.524 0) (size 1.27 2.54) (layers B.Cu B.Paste B.Mask))
  (pad 2 smd rect (at 1.524 0) (size 1.27 2.54) (layers B.Cu B.Paste B.Mask)))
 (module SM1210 (layer B.Cu) (at 207.01 164.084)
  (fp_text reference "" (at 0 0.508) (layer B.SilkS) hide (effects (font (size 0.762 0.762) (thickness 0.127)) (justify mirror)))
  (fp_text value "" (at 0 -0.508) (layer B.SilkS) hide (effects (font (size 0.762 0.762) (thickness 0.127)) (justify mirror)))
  (pad 1 smd rect (at -1.524 0) (size 1.27 2.54) (layers B.Cu B.Paste B.Mask))
  (pad 2 smd rect (at 1.524 0) (size 1.27 2.54) (layers B.Cu B.Paste B.Mask)))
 (gr_line (start 186.69 197.612) (end 186.69 140.716) (angle 90) (layer Edge.Cuts) (width 0.1))
 (gr_line (start 217.17 197.612) (end 186.69 197.612) (angle 90) (layer Edge.Cuts) (width 0.1))
 (gr_line (start 217.17 140.716) (end 217.17 197.612) (angle 90) (layer Edge.Cuts) (width 0.1))
 (gr_line (start 186.69 140.716) (end 217.17 140.716) (angle 90) (layer Edge.Cuts) (width 0.1))
 (segment (start 204.089 170.13936) (end 210.01736 170.13936) (width 0.254) (layer F.Cu) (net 34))
 (segment (start 210.01736 170.13936) (end 212.852 172.974) (width 0.254) (layer F.Cu) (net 34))
 (segment (start 199.38492 185.05424) (end 192.89776 185.05424) (width 0.254) (layer F.Cu) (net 2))
 (segment (start 192.89776 185.05424) (end 191.008 186.944) (width 0.254) (layer F.Cu) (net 2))
 (segment (start 199.38492 184.404) (end 191.008 184.404) (width 0.254) (layer F.Cu) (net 1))
 (segment (start 199.38492 183.75376) (end 192.89776 183.75376) (width 0.254) (layer F.Cu) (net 8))
 (segment (start 192.89776 183.75376) (end 191.008 181.864) (width 0.254) (layer F.Cu) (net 8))
 (segment (start 199.38492 183.10352) (end 194.78752 183.10352) (width 0.254) (layer F.Cu) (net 7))
 (segment (start 194.78752 183.10352) (end 191.008 179.324) (width 0.254) (layer F.Cu) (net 7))
 (segment (start 199.38492 182.45328) (end 196.67728 182.45328) (width 0.254) (layer F.Cu) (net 6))
 (segment (start 196.67728 182.45328) (end 191.008 176.784) (width 0.254) (layer F.Cu) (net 6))
 (segment (start 204.98308 182.45328) (end 207.18272 182.45328) (width 0.254) (layer F.Cu) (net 14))
 (segment (start 207.18272 182.45328) (end 212.852 176.784) (width 0.254) (layer F.Cu) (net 14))
 (segment (start 204.089 169.48912) (end 211.90712 169.48912) (width 0.254) (layer F.Cu) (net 33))
 (segment (start 211.90712 169.48912) (end 212.852 170.434) (width 0.254) (layer F.Cu) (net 33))
 (segment (start 204.089 168.83888) (end 211.90712 168.83888) (width 0.254) (layer F.Cu) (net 32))
 (segment (start 211.90712 168.83888) (end 212.852 167.894) (width 0.254) (layer F.Cu) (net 32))
 (segment (start 204.089 168.18864) (end 210.01736 168.18864) (width 0.254) (layer F.Cu) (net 31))
 (segment (start 210.01736 168.18864) (end 212.852 165.354) (width 0.254) (layer F.Cu) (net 31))
 (segment (start 199.771 170.13936) (end 193.58864 170.13936) (width 0.254) (layer F.Cu) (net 35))
 (segment (start 193.58864 170.13936) (end 191.008 172.72) (width 0.254) (layer F.Cu) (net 35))
 (segment (start 204.98308 183.10352) (end 209.07248 183.10352) (width 0.254) (layer F.Cu) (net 13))
 (segment (start 209.07248 183.10352) (end 212.852 179.324) (width 0.254) (layer F.Cu) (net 13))
 (segment (start 199.771 169.48912) (end 191.69888 169.48912) (width 0.254) (layer F.Cu) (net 36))
 (segment (start 191.69888 169.48912) (end 191.008 170.18) (width 0.254) (layer F.Cu) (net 36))
 (segment (start 199.771 168.83888) (end 192.20688 168.83888) (width 0.254) (layer F.Cu) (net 37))
 (segment (start 192.20688 168.83888) (end 191.008 167.64) (width 0.254) (layer F.Cu) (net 37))
 (segment (start 199.771 168.18864) (end 194.09664 168.18864) (width 0.254) (layer F.Cu) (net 38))
 (segment (start 194.09664 168.18864) (end 191.008 165.1) (width 0.254) (layer F.Cu) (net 38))
 (segment (start 198.755 148.971) (end 194.183 148.971) (width 0.254) (layer F.Cu) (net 28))
 (segment (start 194.183 148.971) (end 191.008 145.796) (width 0.254) (layer F.Cu) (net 28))
 (segment (start 198.755 147.701) (end 195.453 147.701) (width 0.254) (layer F.Cu) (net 29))
 (segment (start 195.453 147.701) (end 191.008 143.256) (width 0.254) (layer F.Cu) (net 29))
 (segment (start 198.755 150.241) (end 192.913 150.241) (width 0.254) (layer F.Cu) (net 27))
 (segment (start 192.913 150.241) (end 191.008 148.336) (width 0.254) (layer F.Cu) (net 27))
 (segment (start 198.755 151.511) (end 191.643 151.511) (width 0.254) (layer F.Cu) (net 26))
 (segment (start 191.643 151.511) (end 191.008 150.876) (width 0.254) (layer F.Cu) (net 26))
 (segment (start 198.755 152.781) (end 191.643 152.781) (width 0.254) (layer F.Cu) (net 25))
 (segment (start 191.643 152.781) (end 191.008 153.416) (width 0.254) (layer F.Cu) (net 25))
 (segment (start 198.755 154.051) (end 192.913 154.051) (width 0.254) (layer F.Cu) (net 24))
 (segment (start 192.913 154.051) (end 191.008 155.956) (width 0.254) (layer F.Cu) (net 24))
 (segment (start 198.755 155.321) (end 194.183 155.321) (width 0.254) (layer F.Cu) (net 23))
 (segment (start 194.183 155.321) (end 191.008 158.496) (width 0.254) (layer F.Cu) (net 23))
 (segment (start 204.98308 183.75376) (end 210.96224 183.75376) (width 0.254) (layer F.Cu) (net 12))
 (segment (start 210.96224 183.75376) (end 212.852 181.864) (width 0.254) (layer F.Cu) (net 12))
 (segment (start 198.755 156.591) (end 195.453 156.591) (width 0.254) (layer F.Cu) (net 22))
 (segment (start 195.453 156.591) (end 191.008 161.036) (width 0.254) (layer F.Cu) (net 22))
 (segment (start 205.105 156.591) (end 208.407 156.591) (width 0.254) (layer F.Cu) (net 21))
 (segment (start 208.407 156.591) (end 212.852 161.036) (width 0.254) (layer F.Cu) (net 21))
 (segment (start 205.105 155.321) (end 209.677 155.321) (width 0.254) (layer F.Cu) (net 20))
 (segment (start 209.677 155.321) (end 212.852 158.496) (width 0.254) (layer F.Cu) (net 20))
 (segment (start 205.105 154.051) (end 210.947 154.051) (width 0.254) (layer F.Cu) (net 19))
 (segment (start 210.947 154.051) (end 212.852 155.956) (width 0.254) (layer F.Cu) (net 19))
 (segment (start 205.105 152.781) (end 212.217 152.781) (width 0.254) (layer F.Cu) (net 18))
 (segment (start 212.217 152.781) (end 212.852 153.416) (width 0.254) (layer F.Cu) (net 18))
 (segment (start 205.105 151.511) (end 212.217 151.511) (width 0.254) (layer F.Cu) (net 17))
 (segment (start 212.217 151.511) (end 212.852 150.876) (width 0.254) (layer F.Cu) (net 17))
 (segment (start 205.105 150.241) (end 210.947 150.241) (width 0.254) (layer F.Cu) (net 16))
 (segment (start 210.947 150.241) (end 212.852 148.336) (width 0.254) (layer F.Cu) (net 16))
 (segment (start 205.105 148.971) (end 209.677 148.971) (width 0.254) (layer F.Cu) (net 30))
 (segment (start 209.677 148.971) (end 212.852 145.796) (width 0.254) (layer F.Cu) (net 30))
 (segment (start 205.105 147.701) (end 208.407 147.701) (width 0.254) (layer F.Cu) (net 15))
 (segment (start 208.407 147.701) (end 212.852 143.256) (width 0.254) (layer F.Cu) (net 15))
 (segment (start 204.98308 184.404) (end 212.852 184.404) (width 0.254) (layer F.Cu) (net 11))
 (segment (start 204.98308 185.05424) (end 210.96224 185.05424) (width 0.254) (layer F.Cu) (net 10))
 (segment (start 210.96224 185.05424) (end 212.852 186.944) (width 0.254) (layer F.Cu) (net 10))
 (segment (start 204.98308 185.70448) (end 209.07248 185.70448) (width 0.254) (layer F.Cu) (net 9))
 (segment (start 209.07248 185.70448) (end 212.852 189.484) (width 0.254) (layer F.Cu) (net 9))
 (segment (start 204.98308 186.35472) (end 207.18272 186.35472) (width 0.254) (layer F.Cu) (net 5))
 (segment (start 207.18272 186.35472) (end 212.852 192.024) (width 0.254) (layer F.Cu) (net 5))
 (segment (start 199.38492 186.35472) (end 196.67728 186.35472) (width 0.254) (layer F.Cu) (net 4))
 (segment (start 196.67728 186.35472) (end 191.008 192.024) (width 0.254) (layer F.Cu) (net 4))
 (segment (start 199.38492 185.70448) (end 194.78752 185.70448) (width 0.254) (layer F.Cu) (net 3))
 (segment (start 194.78752 185.70448) (end 191.008 189.484) (width 0.254) (layer F.Cu) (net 3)))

